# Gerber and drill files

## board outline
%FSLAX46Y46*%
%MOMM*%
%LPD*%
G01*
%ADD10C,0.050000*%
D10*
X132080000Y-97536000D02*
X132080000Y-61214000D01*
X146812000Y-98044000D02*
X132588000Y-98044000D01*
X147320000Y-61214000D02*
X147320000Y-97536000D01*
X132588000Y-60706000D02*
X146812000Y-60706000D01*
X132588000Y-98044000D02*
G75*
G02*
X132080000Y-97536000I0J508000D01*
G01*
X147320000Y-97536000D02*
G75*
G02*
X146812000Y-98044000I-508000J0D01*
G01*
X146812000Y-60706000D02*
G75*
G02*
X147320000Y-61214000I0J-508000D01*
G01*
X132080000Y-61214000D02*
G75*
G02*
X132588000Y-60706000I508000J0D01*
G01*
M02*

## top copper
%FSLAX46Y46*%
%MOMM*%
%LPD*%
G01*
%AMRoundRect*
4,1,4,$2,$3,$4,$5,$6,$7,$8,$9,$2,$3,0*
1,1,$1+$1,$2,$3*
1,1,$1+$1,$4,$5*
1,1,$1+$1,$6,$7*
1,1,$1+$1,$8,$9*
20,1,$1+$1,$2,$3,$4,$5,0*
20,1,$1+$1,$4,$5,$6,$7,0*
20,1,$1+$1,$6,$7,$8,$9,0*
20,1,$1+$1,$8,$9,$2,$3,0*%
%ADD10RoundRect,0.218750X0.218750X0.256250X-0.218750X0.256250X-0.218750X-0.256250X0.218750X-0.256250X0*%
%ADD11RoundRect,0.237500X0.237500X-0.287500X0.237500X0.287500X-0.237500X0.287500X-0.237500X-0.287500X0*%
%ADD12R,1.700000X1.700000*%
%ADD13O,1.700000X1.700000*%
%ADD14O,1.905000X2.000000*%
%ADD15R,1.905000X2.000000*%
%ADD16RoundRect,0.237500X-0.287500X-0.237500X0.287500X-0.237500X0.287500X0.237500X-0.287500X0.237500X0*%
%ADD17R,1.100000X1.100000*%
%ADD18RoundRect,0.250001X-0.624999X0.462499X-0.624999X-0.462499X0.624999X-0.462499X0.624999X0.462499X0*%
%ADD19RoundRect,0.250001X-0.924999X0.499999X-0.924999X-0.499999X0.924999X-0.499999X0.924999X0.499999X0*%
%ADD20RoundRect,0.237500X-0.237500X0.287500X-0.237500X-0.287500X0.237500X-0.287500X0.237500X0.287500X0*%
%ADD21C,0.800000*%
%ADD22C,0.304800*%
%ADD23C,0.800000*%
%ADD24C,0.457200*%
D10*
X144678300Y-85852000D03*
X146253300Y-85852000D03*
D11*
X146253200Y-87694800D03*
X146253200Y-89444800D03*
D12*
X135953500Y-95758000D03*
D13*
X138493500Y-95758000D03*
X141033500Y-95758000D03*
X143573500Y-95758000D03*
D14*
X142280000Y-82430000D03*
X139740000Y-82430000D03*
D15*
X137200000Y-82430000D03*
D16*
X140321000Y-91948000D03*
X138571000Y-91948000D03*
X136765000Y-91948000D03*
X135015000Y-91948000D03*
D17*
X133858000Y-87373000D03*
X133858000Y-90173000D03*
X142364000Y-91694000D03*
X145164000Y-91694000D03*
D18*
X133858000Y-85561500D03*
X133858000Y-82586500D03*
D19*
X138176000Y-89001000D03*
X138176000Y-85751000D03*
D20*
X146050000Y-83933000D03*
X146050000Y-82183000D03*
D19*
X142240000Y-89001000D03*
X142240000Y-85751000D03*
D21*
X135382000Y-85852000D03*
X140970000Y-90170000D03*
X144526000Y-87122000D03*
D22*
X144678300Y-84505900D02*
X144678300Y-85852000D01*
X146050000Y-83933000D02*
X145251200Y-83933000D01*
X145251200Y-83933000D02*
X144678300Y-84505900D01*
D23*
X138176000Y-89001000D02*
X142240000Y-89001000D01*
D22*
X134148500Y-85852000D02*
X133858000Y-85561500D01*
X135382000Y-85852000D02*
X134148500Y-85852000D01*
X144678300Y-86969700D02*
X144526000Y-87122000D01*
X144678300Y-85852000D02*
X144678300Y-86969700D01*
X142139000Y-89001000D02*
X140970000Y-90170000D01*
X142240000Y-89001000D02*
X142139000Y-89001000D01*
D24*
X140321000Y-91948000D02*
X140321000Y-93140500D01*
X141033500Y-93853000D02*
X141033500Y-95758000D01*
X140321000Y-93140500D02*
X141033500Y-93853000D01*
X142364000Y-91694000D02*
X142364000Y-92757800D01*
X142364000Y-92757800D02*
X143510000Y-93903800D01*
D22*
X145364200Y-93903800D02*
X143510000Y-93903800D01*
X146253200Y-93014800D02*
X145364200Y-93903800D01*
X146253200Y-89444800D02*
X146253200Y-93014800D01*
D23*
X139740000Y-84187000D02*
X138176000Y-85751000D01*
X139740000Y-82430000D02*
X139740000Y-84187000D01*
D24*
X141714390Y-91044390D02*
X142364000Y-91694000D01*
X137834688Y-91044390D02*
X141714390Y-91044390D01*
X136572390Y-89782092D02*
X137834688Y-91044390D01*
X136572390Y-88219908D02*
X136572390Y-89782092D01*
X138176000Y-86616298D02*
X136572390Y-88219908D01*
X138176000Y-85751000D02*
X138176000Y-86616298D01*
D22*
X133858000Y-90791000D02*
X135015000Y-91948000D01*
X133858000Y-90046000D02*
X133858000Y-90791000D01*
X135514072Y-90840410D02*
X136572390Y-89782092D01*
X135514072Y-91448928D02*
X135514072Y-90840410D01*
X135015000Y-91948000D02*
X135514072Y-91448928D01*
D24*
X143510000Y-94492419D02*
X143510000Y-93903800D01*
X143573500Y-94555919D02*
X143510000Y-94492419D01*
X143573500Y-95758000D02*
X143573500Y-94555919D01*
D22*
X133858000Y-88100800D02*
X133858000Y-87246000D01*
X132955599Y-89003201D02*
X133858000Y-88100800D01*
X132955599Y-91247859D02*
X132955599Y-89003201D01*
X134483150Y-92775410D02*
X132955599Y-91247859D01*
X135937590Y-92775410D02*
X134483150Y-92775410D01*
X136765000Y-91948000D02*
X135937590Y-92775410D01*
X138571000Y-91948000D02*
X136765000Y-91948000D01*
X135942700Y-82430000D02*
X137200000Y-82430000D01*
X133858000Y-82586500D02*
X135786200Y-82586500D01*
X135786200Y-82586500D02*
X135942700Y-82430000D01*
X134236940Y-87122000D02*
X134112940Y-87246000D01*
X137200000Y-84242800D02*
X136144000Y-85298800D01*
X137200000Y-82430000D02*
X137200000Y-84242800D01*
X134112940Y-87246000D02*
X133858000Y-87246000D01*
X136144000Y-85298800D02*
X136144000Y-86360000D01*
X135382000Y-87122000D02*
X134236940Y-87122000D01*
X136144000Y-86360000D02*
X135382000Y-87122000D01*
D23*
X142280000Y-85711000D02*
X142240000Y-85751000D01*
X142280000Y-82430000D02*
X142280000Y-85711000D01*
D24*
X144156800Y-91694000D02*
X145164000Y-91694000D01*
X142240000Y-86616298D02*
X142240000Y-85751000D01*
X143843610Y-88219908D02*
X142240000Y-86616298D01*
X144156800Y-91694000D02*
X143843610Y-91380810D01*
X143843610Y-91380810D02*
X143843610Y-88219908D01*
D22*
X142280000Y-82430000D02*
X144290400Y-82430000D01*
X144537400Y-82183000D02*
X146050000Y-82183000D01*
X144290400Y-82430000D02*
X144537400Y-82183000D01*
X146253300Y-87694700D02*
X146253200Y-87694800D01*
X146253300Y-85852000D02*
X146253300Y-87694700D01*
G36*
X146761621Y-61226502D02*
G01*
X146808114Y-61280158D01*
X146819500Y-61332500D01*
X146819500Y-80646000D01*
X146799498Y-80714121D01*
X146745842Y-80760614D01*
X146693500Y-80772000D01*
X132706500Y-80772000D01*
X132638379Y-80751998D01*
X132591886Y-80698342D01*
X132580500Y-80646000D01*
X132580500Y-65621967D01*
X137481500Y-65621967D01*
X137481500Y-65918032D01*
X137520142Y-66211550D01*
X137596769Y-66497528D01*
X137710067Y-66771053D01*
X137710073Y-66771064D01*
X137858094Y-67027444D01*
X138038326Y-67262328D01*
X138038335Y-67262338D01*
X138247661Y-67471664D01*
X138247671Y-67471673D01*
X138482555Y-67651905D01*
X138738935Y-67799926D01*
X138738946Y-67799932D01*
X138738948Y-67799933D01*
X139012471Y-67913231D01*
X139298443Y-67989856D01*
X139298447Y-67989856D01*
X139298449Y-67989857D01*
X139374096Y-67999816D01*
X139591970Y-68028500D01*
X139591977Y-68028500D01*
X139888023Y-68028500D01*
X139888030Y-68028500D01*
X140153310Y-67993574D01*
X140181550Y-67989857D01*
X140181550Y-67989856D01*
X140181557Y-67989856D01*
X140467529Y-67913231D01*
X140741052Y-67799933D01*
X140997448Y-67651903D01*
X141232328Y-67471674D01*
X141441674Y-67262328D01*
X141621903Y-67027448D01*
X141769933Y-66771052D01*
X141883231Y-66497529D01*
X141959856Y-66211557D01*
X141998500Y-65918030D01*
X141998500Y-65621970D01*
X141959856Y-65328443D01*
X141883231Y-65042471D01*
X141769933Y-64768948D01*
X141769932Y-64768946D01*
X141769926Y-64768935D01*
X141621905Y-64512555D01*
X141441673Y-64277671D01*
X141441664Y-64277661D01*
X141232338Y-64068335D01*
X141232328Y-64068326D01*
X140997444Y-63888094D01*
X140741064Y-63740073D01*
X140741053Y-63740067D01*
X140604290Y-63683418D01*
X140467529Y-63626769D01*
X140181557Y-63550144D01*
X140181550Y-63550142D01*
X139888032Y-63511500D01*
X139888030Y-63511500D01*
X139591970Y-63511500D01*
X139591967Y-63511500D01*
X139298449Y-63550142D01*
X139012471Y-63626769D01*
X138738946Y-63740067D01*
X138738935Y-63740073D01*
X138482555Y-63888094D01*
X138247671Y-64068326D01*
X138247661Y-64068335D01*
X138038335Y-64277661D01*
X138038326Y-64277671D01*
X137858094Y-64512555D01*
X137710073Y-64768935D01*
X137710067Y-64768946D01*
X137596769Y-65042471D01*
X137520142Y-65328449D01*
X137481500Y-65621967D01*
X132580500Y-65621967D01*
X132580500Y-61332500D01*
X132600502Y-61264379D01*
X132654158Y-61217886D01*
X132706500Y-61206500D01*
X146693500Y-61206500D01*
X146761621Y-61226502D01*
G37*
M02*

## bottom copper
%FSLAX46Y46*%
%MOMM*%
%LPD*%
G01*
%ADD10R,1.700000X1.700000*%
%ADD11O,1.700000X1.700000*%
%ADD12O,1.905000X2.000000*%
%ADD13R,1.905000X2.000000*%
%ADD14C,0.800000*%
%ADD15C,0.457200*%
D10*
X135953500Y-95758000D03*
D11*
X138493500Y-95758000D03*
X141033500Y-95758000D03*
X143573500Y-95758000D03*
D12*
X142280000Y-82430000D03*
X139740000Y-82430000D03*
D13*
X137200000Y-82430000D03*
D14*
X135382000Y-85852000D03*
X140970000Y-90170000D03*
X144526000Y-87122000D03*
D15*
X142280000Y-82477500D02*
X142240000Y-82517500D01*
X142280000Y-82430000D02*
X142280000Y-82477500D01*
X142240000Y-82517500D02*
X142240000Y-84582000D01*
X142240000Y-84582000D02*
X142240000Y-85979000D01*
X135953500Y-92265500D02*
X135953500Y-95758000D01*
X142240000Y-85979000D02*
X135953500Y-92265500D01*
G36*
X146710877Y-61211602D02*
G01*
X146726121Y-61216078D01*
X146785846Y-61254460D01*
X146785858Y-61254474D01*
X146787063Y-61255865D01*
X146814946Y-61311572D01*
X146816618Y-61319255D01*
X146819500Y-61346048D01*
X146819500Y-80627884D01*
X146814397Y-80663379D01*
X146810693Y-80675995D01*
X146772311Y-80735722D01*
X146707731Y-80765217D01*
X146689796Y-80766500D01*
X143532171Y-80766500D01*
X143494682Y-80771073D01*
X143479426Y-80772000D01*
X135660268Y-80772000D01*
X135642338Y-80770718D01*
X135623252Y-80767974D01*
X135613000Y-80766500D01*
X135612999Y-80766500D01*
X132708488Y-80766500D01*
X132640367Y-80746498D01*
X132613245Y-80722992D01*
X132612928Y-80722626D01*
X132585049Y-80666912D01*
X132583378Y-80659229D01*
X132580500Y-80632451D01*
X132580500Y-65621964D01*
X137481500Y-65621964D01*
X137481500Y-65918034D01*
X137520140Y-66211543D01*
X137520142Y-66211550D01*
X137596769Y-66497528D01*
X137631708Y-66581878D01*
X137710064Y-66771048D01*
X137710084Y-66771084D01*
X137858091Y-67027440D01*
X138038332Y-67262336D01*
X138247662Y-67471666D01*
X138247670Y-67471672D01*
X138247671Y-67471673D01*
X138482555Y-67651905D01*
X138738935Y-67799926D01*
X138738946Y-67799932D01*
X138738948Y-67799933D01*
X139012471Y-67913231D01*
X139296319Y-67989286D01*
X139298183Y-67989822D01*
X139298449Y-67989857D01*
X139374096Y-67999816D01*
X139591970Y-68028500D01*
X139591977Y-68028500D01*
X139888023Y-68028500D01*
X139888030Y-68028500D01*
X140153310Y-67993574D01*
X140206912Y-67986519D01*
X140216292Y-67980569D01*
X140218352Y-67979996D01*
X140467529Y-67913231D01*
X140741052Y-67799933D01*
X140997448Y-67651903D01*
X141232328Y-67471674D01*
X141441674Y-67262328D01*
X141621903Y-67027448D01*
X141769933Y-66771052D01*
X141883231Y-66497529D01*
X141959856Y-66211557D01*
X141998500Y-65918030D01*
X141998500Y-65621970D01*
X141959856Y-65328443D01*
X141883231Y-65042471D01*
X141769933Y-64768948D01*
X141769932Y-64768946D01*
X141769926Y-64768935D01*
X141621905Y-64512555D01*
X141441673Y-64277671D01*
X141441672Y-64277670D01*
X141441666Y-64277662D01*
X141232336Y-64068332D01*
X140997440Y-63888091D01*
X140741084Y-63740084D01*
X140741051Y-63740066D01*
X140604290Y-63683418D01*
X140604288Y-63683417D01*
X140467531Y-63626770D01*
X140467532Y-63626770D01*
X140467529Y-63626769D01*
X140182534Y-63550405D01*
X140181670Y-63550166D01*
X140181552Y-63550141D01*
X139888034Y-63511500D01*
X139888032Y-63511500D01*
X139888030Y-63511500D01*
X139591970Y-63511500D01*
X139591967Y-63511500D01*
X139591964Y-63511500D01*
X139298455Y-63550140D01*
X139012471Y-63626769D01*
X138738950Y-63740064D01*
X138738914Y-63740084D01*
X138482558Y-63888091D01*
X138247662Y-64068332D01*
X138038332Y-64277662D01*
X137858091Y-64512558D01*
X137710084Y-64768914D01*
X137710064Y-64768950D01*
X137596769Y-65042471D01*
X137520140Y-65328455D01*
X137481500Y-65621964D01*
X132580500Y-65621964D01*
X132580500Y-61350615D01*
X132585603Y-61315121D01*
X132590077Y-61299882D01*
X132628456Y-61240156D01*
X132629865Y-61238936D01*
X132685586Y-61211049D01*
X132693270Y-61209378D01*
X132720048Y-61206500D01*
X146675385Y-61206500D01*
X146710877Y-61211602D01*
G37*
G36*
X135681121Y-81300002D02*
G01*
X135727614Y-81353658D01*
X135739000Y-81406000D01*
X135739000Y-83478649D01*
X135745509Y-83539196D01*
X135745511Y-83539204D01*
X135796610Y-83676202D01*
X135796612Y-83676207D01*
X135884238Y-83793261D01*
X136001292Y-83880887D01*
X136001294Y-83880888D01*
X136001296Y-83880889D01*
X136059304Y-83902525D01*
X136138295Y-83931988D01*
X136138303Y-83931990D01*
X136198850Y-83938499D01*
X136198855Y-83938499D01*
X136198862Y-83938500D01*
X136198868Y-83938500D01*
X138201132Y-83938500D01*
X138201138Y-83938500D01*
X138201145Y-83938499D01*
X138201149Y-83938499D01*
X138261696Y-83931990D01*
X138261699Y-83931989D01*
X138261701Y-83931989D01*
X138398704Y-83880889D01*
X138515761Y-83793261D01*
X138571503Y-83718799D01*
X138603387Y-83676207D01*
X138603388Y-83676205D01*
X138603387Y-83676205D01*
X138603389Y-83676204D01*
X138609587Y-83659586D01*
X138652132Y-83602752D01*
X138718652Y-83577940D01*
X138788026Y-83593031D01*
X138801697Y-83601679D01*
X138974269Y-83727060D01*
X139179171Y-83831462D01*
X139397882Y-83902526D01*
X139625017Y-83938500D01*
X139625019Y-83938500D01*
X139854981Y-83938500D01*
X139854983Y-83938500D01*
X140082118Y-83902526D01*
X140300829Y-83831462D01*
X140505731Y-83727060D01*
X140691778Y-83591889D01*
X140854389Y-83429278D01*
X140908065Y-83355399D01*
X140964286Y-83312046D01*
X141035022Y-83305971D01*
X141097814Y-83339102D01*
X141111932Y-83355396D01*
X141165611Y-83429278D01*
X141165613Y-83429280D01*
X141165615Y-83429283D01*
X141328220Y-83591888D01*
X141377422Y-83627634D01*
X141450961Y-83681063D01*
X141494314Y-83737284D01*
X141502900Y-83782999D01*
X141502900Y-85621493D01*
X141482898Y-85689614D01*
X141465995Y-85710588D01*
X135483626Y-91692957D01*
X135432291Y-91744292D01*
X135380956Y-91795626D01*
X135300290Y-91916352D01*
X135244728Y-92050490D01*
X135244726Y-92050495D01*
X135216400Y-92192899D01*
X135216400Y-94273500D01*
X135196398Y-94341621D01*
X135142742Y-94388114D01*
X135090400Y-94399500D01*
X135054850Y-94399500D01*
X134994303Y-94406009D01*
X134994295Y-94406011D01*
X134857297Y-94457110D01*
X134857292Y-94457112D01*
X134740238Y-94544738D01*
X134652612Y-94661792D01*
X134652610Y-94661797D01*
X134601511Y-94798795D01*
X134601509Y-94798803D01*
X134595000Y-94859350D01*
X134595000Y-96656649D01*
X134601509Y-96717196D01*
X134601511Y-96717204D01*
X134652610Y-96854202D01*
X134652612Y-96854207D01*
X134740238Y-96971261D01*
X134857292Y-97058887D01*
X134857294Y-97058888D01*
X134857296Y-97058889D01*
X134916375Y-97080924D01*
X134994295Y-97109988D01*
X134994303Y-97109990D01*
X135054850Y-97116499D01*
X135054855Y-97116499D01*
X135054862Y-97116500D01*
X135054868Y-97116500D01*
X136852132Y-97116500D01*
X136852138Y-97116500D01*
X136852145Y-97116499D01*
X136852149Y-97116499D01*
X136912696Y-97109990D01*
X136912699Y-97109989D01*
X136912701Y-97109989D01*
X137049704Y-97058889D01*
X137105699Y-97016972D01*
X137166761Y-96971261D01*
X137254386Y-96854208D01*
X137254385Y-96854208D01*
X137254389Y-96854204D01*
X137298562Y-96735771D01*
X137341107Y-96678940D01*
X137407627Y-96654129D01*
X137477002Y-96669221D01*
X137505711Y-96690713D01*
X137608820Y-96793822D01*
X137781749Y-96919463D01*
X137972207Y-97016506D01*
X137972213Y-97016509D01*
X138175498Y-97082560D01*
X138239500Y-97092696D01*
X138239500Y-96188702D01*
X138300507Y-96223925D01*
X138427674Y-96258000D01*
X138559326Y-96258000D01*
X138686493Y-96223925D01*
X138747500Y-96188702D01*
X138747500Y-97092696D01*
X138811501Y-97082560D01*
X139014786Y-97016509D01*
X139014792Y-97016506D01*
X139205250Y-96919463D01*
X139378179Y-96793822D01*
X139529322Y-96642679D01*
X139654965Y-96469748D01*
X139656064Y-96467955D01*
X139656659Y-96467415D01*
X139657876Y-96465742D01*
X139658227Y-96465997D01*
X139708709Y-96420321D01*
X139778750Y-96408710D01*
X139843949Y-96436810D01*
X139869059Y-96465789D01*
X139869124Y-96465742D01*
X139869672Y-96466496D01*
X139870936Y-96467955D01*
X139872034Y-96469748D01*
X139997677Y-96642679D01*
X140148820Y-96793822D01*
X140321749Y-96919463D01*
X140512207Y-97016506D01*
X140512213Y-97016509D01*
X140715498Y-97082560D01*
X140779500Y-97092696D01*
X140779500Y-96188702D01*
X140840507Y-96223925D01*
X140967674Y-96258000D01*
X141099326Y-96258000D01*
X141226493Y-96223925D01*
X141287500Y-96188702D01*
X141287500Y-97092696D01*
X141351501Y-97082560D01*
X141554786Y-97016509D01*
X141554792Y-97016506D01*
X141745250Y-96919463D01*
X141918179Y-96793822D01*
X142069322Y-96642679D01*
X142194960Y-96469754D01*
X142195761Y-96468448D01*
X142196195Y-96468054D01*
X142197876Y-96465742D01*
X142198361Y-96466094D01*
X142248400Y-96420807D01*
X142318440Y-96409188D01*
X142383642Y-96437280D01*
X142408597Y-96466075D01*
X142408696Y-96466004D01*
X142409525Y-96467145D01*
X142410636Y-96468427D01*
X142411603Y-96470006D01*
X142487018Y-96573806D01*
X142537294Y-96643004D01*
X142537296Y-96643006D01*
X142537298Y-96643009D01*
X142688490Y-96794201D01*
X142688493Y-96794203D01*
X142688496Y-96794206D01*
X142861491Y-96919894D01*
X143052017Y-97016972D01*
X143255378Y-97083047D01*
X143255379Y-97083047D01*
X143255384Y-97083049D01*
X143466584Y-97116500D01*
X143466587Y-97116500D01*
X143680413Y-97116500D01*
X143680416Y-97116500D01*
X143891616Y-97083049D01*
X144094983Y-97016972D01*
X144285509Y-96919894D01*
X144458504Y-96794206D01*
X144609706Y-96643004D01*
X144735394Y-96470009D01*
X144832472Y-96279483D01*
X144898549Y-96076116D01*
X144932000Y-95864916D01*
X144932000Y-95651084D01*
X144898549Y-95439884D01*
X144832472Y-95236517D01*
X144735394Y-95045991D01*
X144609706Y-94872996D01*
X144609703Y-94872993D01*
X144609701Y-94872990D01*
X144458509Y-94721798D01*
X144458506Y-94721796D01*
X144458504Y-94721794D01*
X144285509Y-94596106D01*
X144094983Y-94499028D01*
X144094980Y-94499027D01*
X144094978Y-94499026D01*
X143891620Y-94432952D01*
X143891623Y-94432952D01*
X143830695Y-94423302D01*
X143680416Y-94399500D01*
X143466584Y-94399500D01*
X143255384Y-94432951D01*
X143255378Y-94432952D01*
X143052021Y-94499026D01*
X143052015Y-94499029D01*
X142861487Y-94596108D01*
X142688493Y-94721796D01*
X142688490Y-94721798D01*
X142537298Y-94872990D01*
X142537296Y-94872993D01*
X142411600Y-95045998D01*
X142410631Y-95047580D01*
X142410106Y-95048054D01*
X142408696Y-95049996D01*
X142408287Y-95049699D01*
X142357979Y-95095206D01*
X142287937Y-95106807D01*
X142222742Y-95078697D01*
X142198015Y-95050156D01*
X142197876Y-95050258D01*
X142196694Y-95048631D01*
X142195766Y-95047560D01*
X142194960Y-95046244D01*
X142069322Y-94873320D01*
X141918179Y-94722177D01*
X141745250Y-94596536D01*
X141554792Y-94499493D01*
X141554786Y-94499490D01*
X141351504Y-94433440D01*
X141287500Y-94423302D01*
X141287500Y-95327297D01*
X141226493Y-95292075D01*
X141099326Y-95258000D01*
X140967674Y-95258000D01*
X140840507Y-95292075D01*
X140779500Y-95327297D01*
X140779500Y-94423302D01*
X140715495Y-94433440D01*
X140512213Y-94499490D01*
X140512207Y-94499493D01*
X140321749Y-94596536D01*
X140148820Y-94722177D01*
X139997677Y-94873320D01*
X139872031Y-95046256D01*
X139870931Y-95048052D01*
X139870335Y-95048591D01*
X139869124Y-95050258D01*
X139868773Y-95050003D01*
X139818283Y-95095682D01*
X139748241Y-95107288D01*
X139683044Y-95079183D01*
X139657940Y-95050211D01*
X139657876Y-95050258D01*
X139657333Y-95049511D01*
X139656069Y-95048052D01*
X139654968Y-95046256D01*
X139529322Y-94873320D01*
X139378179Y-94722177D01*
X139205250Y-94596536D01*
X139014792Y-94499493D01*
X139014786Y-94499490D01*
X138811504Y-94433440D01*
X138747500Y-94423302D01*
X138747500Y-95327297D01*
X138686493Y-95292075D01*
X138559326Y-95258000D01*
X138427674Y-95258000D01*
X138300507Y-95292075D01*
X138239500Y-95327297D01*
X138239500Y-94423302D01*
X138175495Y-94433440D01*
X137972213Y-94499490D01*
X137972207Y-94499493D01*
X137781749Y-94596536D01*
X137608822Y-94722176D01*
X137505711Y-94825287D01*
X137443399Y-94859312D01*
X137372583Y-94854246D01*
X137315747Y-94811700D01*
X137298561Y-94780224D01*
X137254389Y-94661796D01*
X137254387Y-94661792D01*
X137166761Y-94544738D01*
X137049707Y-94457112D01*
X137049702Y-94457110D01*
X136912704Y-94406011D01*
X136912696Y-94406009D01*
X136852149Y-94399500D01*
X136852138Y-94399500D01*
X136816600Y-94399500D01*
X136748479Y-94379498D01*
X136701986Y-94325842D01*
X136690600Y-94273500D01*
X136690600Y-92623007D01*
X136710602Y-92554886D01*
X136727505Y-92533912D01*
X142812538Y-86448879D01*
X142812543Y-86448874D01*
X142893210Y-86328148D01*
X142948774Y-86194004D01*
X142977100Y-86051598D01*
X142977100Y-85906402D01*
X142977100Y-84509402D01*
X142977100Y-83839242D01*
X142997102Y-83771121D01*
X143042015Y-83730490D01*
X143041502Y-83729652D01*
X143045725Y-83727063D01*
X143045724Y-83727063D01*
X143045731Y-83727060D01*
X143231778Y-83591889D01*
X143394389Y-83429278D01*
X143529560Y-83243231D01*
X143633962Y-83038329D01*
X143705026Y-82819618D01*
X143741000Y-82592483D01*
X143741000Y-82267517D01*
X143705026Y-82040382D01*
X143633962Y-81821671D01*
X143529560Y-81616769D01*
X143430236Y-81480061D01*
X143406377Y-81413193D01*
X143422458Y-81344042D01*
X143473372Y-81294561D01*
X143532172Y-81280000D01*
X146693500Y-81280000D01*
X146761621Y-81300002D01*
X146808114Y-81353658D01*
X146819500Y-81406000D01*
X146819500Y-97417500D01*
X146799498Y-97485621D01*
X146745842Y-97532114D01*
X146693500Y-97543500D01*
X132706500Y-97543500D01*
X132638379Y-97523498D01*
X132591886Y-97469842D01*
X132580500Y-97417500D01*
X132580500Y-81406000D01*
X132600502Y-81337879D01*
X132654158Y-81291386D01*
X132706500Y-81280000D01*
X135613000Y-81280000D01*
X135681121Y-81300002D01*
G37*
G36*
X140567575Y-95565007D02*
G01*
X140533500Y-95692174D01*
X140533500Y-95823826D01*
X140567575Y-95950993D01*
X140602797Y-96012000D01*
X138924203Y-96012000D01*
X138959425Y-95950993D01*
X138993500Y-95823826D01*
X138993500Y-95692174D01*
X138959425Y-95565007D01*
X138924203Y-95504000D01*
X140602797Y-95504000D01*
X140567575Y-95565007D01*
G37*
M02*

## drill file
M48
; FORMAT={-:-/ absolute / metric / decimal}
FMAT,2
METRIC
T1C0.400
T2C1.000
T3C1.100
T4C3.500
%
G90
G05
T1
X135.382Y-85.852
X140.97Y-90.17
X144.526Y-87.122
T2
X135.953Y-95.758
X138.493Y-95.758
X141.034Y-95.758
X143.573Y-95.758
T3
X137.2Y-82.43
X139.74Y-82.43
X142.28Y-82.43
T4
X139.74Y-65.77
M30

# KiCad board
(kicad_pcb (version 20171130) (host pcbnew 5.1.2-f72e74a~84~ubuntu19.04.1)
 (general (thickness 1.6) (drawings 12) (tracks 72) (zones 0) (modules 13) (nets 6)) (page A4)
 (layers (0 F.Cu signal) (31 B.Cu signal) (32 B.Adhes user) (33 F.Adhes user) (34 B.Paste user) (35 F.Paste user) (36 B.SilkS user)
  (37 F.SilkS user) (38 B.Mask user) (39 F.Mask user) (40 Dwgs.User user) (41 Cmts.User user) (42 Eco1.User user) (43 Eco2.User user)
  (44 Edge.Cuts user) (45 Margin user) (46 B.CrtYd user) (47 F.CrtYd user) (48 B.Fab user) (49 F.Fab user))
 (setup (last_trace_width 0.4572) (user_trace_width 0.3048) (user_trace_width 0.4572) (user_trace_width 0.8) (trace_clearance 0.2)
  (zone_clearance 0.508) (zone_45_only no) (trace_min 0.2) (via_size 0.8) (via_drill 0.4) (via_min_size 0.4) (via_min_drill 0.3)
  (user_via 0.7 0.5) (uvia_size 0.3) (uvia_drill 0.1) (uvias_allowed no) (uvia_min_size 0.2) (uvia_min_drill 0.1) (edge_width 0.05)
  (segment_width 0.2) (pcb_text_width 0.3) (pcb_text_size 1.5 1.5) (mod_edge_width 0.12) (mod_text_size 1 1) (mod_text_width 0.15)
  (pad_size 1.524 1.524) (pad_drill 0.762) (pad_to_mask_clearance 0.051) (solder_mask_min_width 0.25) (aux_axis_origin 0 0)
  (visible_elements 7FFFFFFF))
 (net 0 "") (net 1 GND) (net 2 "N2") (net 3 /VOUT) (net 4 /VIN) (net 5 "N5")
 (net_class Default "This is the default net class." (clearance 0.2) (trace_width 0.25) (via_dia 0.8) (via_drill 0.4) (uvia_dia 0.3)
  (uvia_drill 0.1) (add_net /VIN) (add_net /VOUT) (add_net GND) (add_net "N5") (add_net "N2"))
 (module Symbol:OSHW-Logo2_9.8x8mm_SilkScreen (layer B.Cu) (at 139.7 72.39 180)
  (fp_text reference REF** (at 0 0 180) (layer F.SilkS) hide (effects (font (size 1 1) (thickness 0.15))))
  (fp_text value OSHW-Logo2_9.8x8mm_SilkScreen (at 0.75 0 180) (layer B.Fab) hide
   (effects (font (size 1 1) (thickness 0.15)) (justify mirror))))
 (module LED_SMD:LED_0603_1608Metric (layer F.Cu) (at 145.4658 85.852 180)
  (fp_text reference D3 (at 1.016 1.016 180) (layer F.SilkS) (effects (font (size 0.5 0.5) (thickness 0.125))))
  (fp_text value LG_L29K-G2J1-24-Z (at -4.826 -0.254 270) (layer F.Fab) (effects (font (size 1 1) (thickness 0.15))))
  (pad 2 smd roundrect (at 0.7875 0 180) (size 0.875 0.95) (layers F.Cu F.Paste F.Mask) (roundrect_rratio 0.25) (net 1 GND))
  (pad 1 smd roundrect (at -0.7875 0 180) (size 0.875 0.95) (layers F.Cu F.Paste F.Mask) (roundrect_rratio 0.25) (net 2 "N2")))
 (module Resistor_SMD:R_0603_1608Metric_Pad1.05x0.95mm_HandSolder (layer F.Cu) (at 146.2532 88.5698 90)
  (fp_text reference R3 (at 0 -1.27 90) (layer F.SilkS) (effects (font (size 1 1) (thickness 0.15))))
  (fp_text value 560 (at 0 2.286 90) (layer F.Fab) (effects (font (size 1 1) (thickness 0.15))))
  (pad 2 smd roundrect (at 0.875 0 90) (size 1.05 0.95) (layers F.Cu F.Paste F.Mask) (roundrect_rratio 0.25) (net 2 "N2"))
  (pad 1 smd roundrect (at -0.875 0 90) (size 1.05 0.95) (layers F.Cu F.Paste F.Mask) (roundrect_rratio 0.25) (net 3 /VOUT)))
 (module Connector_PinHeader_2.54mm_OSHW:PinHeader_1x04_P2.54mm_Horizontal (layer F.Cu) (at 135.9535 95.758 90)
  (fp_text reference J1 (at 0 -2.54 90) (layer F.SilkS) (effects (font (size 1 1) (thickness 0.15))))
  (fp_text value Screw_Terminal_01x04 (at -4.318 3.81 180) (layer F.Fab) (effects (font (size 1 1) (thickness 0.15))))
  (pad 1 thru_hole rect (at 0 0 90) (size 1.7 1.7) (drill 1) (layers *.Cu *.Mask) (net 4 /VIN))
  (pad 2 thru_hole oval (at 0 2.54 90) (size 1.7 1.7) (drill 1) (layers *.Cu *.Mask) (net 1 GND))
  (pad 3 thru_hole oval (at 0 5.08 90) (size 1.7 1.7) (drill 1) (layers *.Cu *.Mask) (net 1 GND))
  (pad 4 thru_hole oval (at 0 7.62 90) (size 1.7 1.7) (drill 1) (layers *.Cu *.Mask) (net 3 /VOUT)))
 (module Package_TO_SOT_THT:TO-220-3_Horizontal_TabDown (layer F.Cu) (at 137.2 82.43)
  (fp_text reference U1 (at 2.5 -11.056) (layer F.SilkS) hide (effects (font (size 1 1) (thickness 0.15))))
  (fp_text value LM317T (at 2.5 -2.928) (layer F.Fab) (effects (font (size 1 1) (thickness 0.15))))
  (pad 3 thru_hole oval (at 5.08 0) (size 1.905 2) (drill 1.1) (layers *.Cu *.Mask) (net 4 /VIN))
  (pad 2 thru_hole oval (at 2.54 0) (size 1.905 2) (drill 1.1) (layers *.Cu *.Mask) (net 3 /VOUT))
  (pad 1 thru_hole rect (at 0 0) (size 1.905 2) (drill 1.1) (layers *.Cu *.Mask) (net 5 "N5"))
  (pad "" np_thru_hole oval (at 2.54 -16.66) (size 3.5 3.5) (drill 3.5) (layers *.Cu *.Mask)))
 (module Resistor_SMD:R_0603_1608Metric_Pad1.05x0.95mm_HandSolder (layer F.Cu) (at 139.446 91.948)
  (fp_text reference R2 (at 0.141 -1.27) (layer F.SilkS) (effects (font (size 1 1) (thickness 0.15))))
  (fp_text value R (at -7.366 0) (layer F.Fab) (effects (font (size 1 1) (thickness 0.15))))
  (pad 2 smd roundrect (at 0.875 0) (size 1.05 0.95) (layers F.Cu F.Paste F.Mask) (roundrect_rratio 0.25) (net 1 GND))
  (pad 1 smd roundrect (at -0.875 0) (size 1.05 0.95) (layers F.Cu F.Paste F.Mask) (roundrect_rratio 0.25) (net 5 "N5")))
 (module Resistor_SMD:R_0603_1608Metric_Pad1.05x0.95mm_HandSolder (layer F.Cu) (at 135.89 91.948)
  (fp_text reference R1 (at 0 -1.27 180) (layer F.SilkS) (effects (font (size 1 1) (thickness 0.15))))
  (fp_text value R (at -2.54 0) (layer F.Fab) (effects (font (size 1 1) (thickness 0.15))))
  (pad 2 smd roundrect (at 0.875 0) (size 1.05 0.95) (layers F.Cu F.Paste F.Mask) (roundrect_rratio 0.25) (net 5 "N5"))
  (pad 1 smd roundrect (at -0.875 0) (size 1.05 0.95) (layers F.Cu F.Paste F.Mask) (roundrect_rratio 0.25) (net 3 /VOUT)))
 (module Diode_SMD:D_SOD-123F (layer F.Cu) (at 133.858 88.773 90)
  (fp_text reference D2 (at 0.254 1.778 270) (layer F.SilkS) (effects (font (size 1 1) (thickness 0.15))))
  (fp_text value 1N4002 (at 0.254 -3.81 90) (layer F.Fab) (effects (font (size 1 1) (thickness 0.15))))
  (pad 2 smd rect (at 1.4 0 90) (size 1.1 1.1) (layers F.Cu F.Paste F.Mask) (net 5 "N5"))
  (pad 1 smd rect (at -1.4 0 90) (size 1.1 1.1) (layers F.Cu F.Paste F.Mask) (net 3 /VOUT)))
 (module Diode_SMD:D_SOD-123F (layer F.Cu) (at 143.764 91.694 180)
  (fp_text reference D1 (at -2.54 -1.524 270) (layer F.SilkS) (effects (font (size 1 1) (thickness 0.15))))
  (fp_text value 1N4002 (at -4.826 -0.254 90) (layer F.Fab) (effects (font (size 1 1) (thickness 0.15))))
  (pad 2 smd rect (at 1.4 0 180) (size 1.1 1.1) (layers F.Cu F.Paste F.Mask) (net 3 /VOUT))
  (pad 1 smd rect (at -1.4 0 180) (size 1.1 1.1) (layers F.Cu F.Paste F.Mask) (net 4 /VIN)))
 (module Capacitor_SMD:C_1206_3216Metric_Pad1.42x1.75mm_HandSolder (layer F.Cu) (at 133.858 84.074 270)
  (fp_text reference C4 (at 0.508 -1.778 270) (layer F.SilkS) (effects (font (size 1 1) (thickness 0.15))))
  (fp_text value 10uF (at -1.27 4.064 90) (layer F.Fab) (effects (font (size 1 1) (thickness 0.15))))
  (pad 2 smd roundrect (at 1.4875 0 270) (size 1.425 1.75) (layers F.Cu F.Paste F.Mask) (roundrect_rratio 0.175439) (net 1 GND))
  (pad 1 smd roundrect (at -1.4875 0 270) (size 1.425 1.75) (layers F.Cu F.Paste F.Mask) (roundrect_rratio 0.175439) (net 5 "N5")))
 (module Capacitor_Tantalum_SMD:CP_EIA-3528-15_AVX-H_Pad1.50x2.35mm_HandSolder (layer F.Cu) (at 138.176 87.376 270)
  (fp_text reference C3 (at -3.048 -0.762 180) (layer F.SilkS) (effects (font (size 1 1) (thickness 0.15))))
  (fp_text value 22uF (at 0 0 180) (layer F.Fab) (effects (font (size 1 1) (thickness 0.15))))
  (pad 2 smd roundrect (at 1.625 0 270) (size 1.5 2.35) (layers F.Cu F.Paste F.Mask) (roundrect_rratio 0.166667) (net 1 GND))
  (pad 1 smd roundrect (at -1.625 0 270) (size 1.5 2.35) (layers F.Cu F.Paste F.Mask) (roundrect_rratio 0.166667) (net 3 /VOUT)))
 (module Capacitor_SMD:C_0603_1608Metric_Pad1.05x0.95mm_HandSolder (layer F.Cu) (at 146.05 83.058 270)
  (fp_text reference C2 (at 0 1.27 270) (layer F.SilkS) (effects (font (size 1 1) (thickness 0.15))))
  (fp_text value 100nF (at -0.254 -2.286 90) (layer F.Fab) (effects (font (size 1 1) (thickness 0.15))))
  (pad 2 smd roundrect (at 0.875 0 270) (size 1.05 0.95) (layers F.Cu F.Paste F.Mask) (roundrect_rratio 0.25) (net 1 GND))
  (pad 1 smd roundrect (at -0.875 0 270) (size 1.05 0.95) (layers F.Cu F.Paste F.Mask) (roundrect_rratio 0.25) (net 4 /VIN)))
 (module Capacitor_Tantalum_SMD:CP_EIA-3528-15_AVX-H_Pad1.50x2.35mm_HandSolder (layer F.Cu) (at 142.24 87.376 270)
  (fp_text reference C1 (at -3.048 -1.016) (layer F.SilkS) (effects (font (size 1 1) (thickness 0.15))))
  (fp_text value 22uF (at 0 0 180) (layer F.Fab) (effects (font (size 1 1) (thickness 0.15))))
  (pad 2 smd roundrect (at 1.625 0 270) (size 1.5 2.35) (layers F.Cu F.Paste F.Mask) (roundrect_rratio 0.166667) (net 1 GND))
  (pad 1 smd roundrect (at -1.625 0 270) (size 1.5 2.35) (layers F.Cu F.Paste F.Mask) (roundrect_rratio 0.166667) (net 4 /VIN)))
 (gr_line (start 132.08 97.536) (end 132.08 61.214) (layer Edge.Cuts) (width 0.05))
 (gr_line (start 146.812 98.044) (end 132.588 98.044) (layer Edge.Cuts) (width 0.05))
 (gr_line (start 147.32 61.214) (end 147.32 97.536) (layer Edge.Cuts) (width 0.05))
 (gr_line (start 132.588 60.706) (end 146.812 60.706) (layer Edge.Cuts) (width 0.05))
 (gr_arc (start 132.588 97.536) (end 132.08 97.536) (angle -90) (layer Edge.Cuts) (width 0.05))
 (gr_arc (start 146.812 97.536) (end 146.812 98.044) (angle -90) (layer Edge.Cuts) (width 0.05))
 (gr_arc (start 146.812 61.214) (end 147.32 61.214) (angle -90) (layer Edge.Cuts) (width 0.05))
 (gr_arc (start 132.588 61.214) (end 132.588 60.706) (angle -90) (layer Edge.Cuts) (width 0.05))
 (segment (start 144.6783 84.5059) (end 144.6783 85.852) (width 0.3048) (layer F.Cu) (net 1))
 (segment (start 146.05 83.933) (end 145.2512 83.933) (width 0.3048) (layer F.Cu) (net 1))
 (segment (start 145.2512 83.933) (end 144.6783 84.5059) (width 0.3048) (layer F.Cu) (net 1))
 (segment (start 138.176 89.001) (end 142.24 89.001) (width 0.8) (layer F.Cu) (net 1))
 (via (at 135.382 85.852) (size 0.8) (drill 0.4) (layers F.Cu B.Cu) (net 1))
 (segment (start 134.1485 85.852) (end 133.858 85.5615) (width 0.3048) (layer F.Cu) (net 1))
 (segment (start 135.382 85.852) (end 134.1485 85.852) (width 0.3048) (layer F.Cu) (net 1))
 (via (at 140.97 90.17) (size 0.8) (drill 0.4) (layers F.Cu B.Cu) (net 1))
 (via (at 144.526 87.122) (size 0.8) (drill 0.4) (layers F.Cu B.Cu) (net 1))
 (segment (start 144.6783 86.9697) (end 144.526 87.122) (width 0.3048) (layer F.Cu) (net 1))
 (segment (start 144.6783 85.852) (end 144.6783 86.9697) (width 0.3048) (layer F.Cu) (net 1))
 (segment (start 142.139 89.001) (end 140.97 90.17) (width 0.3048) (layer F.Cu) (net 1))
 (segment (start 142.24 89.001) (end 142.139 89.001) (width 0.3048) (layer F.Cu) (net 1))
 (segment (start 140.321 91.948) (end 140.321 93.1405) (width 0.4572) (layer F.Cu) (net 1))
 (segment (start 141.0335 93.853) (end 141.0335 95.758) (width 0.4572) (layer F.Cu) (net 1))
 (segment (start 140.321 93.1405) (end 141.0335 93.853) (width 0.4572) (layer F.Cu) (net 1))
 (segment (start 142.364 91.694) (end 142.364 92.7578) (width 0.4572) (layer F.Cu) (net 3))
 (segment (start 142.364 92.7578) (end 143.51 93.9038) (width 0.4572) (layer F.Cu) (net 3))
 (segment (start 145.3642 93.9038) (end 143.51 93.9038) (width 0.3048) (layer F.Cu) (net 3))
 (segment (start 146.2532 93.0148) (end 145.3642 93.9038) (width 0.3048) (layer F.Cu) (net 3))
 (segment (start 146.2532 89.4448) (end 146.2532 93.0148) (width 0.3048) (layer F.Cu) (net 3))
 (segment (start 139.74 84.187) (end 138.176 85.751) (width 0.8) (layer F.Cu) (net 3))
 (segment (start 139.74 82.43) (end 139.74 84.187) (width 0.8) (layer F.Cu) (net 3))
 (segment (start 141.71439 91.04439) (end 142.364 91.694) (width 0.4572) (layer F.Cu) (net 3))
 (segment (start 137.834688 91.04439) (end 141.71439 91.04439) (width 0.4572) (layer F.Cu) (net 3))
 (segment (start 136.57239 89.782092) (end 137.834688 91.04439) (width 0.4572) (layer F.Cu) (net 3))
 (segment (start 136.57239 88.219908) (end 136.57239 89.782092) (width 0.4572) (layer F.Cu) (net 3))
 (segment (start 138.176 86.616298) (end 136.57239 88.219908) (width 0.4572) (layer F.Cu) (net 3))
 (segment (start 138.176 85.751) (end 138.176 86.616298) (width 0.4572) (layer F.Cu) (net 3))
 (segment (start 133.858 90.791) (end 135.015 91.948) (width 0.3048) (layer F.Cu) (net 3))
 (segment (start 133.858 90.046) (end 133.858 90.791) (width 0.3048) (layer F.Cu) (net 3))
 (segment (start 135.514072 90.84041) (end 136.57239 89.782092) (width 0.3048) (layer F.Cu) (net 3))
 (segment (start 135.514072 91.448928) (end 135.514072 90.84041) (width 0.3048) (layer F.Cu) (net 3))
 (segment (start 135.015 91.948) (end 135.514072 91.448928) (width 0.3048) (layer F.Cu) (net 3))
 (segment (start 143.51 94.492419) (end 143.51 93.9038) (width 0.4572) (layer F.Cu) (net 3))
 (segment (start 143.5735 94.555919) (end 143.51 94.492419) (width 0.4572) (layer F.Cu) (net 3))
 (segment (start 143.5735 95.758) (end 143.5735 94.555919) (width 0.4572) (layer F.Cu) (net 3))
 (segment (start 133.858 88.1008) (end 133.858 87.246) (width 0.3048) (layer F.Cu) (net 5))
 (segment (start 132.955599 89.003201) (end 133.858 88.1008) (width 0.3048) (layer F.Cu) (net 5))
 (segment (start 132.955599 91.247859) (end 132.955599 89.003201) (width 0.3048) (layer F.Cu) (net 5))
 (segment (start 134.48315 92.77541) (end 132.955599 91.247859) (width 0.3048) (layer F.Cu) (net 5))
 (segment (start 135.93759 92.77541) (end 134.48315 92.77541) (width 0.3048) (layer F.Cu) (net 5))
 (segment (start 136.765 91.948) (end 135.93759 92.77541) (width 0.3048) (layer F.Cu) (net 5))
 (segment (start 138.571 91.948) (end 136.765 91.948) (width 0.3048) (layer F.Cu) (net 5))
 (segment (start 135.9427 82.43) (end 137.2 82.43) (width 0.3048) (layer F.Cu) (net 5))
 (segment (start 133.858 82.5865) (end 135.7862 82.5865) (width 0.3048) (layer F.Cu) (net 5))
 (segment (start 135.7862 82.5865) (end 135.9427 82.43) (width 0.3048) (layer F.Cu) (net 5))
 (segment (start 134.23694 87.122) (end 134.11294 87.246) (width 0.3048) (layer F.Cu) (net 5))
 (segment (start 137.2 84.2428) (end 136.144 85.2988) (width 0.3048) (layer F.Cu) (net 5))
 (segment (start 137.2 82.43) (end 137.2 84.2428) (width 0.3048) (layer F.Cu) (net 5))
 (segment (start 134.11294 87.246) (end 133.858 87.246) (width 0.3048) (layer F.Cu) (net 5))
 (segment (start 136.144 85.2988) (end 136.144 86.36) (width 0.3048) (layer F.Cu) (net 5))
 (segment (start 135.382 87.122) (end 134.23694 87.122) (width 0.3048) (layer F.Cu) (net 5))
 (segment (start 136.144 86.36) (end 135.382 87.122) (width 0.3048) (layer F.Cu) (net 5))
 (segment (start 142.28 85.711) (end 142.24 85.751) (width 0.8) (layer F.Cu) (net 4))
 (segment (start 142.28 82.43) (end 142.28 85.711) (width 0.8) (layer F.Cu) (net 4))
 (segment (start 144.1568 91.694) (end 145.164 91.694) (width 0.4572) (layer F.Cu) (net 4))
 (segment (start 142.24 86.616298) (end 142.24 85.751) (width 0.4572) (layer F.Cu) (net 4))
 (segment (start 143.84361 88.219908) (end 142.24 86.616298) (width 0.4572) (layer F.Cu) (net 4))
 (segment (start 144.1568 91.694) (end 143.84361 91.38081) (width 0.4572) (layer F.Cu) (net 4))
 (segment (start 143.84361 91.38081) (end 143.84361 88.219908) (width 0.4572) (layer F.Cu) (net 4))
 (segment (start 142.28 82.43) (end 144.2904 82.43) (width 0.3048) (layer F.Cu) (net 4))
 (segment (start 144.5374 82.183) (end 146.05 82.183) (width 0.3048) (layer F.Cu) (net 4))
 (segment (start 144.2904 82.43) (end 144.5374 82.183) (width 0.3048) (layer F.Cu) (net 4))
 (segment (start 142.28 82.4775) (end 142.24 82.5175) (width 0.4572) (layer B.Cu) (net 4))
 (segment (start 142.28 82.43) (end 142.28 82.4775) (width 0.4572) (layer B.Cu) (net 4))
 (segment (start 142.24 82.5175) (end 142.24 84.582) (width 0.4572) (layer B.Cu) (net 4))
 (segment (start 142.24 84.582) (end 142.24 85.979) (width 0.4572) (layer B.Cu) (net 4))
 (segment (start 135.9535 92.2655) (end 135.9535 95.758) (width 0.4572) (layer B.Cu) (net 4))
 (segment (start 142.24 85.979) (end 135.9535 92.2655) (width 0.4572) (layer B.Cu) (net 4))
 (segment (start 146.2533 87.6947) (end 146.2532 87.6948) (width 0.3048) (layer F.Cu) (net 2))
 (segment (start 146.2533 85.852) (end 146.2533 87.6947) (width 0.3048) (layer F.Cu) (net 2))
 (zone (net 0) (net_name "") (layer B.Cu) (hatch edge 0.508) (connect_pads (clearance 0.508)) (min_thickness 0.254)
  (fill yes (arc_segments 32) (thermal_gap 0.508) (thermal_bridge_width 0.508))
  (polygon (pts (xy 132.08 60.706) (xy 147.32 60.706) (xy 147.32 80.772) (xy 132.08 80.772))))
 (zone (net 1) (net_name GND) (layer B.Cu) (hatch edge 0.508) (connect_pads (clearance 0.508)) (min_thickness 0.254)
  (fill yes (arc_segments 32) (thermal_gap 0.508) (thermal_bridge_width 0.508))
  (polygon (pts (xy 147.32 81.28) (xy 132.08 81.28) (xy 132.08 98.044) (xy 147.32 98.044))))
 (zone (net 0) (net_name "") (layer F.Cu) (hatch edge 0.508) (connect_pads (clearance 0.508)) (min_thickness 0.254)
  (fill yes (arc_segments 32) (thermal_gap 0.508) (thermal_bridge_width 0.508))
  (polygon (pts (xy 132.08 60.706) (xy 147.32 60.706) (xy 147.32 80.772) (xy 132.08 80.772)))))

